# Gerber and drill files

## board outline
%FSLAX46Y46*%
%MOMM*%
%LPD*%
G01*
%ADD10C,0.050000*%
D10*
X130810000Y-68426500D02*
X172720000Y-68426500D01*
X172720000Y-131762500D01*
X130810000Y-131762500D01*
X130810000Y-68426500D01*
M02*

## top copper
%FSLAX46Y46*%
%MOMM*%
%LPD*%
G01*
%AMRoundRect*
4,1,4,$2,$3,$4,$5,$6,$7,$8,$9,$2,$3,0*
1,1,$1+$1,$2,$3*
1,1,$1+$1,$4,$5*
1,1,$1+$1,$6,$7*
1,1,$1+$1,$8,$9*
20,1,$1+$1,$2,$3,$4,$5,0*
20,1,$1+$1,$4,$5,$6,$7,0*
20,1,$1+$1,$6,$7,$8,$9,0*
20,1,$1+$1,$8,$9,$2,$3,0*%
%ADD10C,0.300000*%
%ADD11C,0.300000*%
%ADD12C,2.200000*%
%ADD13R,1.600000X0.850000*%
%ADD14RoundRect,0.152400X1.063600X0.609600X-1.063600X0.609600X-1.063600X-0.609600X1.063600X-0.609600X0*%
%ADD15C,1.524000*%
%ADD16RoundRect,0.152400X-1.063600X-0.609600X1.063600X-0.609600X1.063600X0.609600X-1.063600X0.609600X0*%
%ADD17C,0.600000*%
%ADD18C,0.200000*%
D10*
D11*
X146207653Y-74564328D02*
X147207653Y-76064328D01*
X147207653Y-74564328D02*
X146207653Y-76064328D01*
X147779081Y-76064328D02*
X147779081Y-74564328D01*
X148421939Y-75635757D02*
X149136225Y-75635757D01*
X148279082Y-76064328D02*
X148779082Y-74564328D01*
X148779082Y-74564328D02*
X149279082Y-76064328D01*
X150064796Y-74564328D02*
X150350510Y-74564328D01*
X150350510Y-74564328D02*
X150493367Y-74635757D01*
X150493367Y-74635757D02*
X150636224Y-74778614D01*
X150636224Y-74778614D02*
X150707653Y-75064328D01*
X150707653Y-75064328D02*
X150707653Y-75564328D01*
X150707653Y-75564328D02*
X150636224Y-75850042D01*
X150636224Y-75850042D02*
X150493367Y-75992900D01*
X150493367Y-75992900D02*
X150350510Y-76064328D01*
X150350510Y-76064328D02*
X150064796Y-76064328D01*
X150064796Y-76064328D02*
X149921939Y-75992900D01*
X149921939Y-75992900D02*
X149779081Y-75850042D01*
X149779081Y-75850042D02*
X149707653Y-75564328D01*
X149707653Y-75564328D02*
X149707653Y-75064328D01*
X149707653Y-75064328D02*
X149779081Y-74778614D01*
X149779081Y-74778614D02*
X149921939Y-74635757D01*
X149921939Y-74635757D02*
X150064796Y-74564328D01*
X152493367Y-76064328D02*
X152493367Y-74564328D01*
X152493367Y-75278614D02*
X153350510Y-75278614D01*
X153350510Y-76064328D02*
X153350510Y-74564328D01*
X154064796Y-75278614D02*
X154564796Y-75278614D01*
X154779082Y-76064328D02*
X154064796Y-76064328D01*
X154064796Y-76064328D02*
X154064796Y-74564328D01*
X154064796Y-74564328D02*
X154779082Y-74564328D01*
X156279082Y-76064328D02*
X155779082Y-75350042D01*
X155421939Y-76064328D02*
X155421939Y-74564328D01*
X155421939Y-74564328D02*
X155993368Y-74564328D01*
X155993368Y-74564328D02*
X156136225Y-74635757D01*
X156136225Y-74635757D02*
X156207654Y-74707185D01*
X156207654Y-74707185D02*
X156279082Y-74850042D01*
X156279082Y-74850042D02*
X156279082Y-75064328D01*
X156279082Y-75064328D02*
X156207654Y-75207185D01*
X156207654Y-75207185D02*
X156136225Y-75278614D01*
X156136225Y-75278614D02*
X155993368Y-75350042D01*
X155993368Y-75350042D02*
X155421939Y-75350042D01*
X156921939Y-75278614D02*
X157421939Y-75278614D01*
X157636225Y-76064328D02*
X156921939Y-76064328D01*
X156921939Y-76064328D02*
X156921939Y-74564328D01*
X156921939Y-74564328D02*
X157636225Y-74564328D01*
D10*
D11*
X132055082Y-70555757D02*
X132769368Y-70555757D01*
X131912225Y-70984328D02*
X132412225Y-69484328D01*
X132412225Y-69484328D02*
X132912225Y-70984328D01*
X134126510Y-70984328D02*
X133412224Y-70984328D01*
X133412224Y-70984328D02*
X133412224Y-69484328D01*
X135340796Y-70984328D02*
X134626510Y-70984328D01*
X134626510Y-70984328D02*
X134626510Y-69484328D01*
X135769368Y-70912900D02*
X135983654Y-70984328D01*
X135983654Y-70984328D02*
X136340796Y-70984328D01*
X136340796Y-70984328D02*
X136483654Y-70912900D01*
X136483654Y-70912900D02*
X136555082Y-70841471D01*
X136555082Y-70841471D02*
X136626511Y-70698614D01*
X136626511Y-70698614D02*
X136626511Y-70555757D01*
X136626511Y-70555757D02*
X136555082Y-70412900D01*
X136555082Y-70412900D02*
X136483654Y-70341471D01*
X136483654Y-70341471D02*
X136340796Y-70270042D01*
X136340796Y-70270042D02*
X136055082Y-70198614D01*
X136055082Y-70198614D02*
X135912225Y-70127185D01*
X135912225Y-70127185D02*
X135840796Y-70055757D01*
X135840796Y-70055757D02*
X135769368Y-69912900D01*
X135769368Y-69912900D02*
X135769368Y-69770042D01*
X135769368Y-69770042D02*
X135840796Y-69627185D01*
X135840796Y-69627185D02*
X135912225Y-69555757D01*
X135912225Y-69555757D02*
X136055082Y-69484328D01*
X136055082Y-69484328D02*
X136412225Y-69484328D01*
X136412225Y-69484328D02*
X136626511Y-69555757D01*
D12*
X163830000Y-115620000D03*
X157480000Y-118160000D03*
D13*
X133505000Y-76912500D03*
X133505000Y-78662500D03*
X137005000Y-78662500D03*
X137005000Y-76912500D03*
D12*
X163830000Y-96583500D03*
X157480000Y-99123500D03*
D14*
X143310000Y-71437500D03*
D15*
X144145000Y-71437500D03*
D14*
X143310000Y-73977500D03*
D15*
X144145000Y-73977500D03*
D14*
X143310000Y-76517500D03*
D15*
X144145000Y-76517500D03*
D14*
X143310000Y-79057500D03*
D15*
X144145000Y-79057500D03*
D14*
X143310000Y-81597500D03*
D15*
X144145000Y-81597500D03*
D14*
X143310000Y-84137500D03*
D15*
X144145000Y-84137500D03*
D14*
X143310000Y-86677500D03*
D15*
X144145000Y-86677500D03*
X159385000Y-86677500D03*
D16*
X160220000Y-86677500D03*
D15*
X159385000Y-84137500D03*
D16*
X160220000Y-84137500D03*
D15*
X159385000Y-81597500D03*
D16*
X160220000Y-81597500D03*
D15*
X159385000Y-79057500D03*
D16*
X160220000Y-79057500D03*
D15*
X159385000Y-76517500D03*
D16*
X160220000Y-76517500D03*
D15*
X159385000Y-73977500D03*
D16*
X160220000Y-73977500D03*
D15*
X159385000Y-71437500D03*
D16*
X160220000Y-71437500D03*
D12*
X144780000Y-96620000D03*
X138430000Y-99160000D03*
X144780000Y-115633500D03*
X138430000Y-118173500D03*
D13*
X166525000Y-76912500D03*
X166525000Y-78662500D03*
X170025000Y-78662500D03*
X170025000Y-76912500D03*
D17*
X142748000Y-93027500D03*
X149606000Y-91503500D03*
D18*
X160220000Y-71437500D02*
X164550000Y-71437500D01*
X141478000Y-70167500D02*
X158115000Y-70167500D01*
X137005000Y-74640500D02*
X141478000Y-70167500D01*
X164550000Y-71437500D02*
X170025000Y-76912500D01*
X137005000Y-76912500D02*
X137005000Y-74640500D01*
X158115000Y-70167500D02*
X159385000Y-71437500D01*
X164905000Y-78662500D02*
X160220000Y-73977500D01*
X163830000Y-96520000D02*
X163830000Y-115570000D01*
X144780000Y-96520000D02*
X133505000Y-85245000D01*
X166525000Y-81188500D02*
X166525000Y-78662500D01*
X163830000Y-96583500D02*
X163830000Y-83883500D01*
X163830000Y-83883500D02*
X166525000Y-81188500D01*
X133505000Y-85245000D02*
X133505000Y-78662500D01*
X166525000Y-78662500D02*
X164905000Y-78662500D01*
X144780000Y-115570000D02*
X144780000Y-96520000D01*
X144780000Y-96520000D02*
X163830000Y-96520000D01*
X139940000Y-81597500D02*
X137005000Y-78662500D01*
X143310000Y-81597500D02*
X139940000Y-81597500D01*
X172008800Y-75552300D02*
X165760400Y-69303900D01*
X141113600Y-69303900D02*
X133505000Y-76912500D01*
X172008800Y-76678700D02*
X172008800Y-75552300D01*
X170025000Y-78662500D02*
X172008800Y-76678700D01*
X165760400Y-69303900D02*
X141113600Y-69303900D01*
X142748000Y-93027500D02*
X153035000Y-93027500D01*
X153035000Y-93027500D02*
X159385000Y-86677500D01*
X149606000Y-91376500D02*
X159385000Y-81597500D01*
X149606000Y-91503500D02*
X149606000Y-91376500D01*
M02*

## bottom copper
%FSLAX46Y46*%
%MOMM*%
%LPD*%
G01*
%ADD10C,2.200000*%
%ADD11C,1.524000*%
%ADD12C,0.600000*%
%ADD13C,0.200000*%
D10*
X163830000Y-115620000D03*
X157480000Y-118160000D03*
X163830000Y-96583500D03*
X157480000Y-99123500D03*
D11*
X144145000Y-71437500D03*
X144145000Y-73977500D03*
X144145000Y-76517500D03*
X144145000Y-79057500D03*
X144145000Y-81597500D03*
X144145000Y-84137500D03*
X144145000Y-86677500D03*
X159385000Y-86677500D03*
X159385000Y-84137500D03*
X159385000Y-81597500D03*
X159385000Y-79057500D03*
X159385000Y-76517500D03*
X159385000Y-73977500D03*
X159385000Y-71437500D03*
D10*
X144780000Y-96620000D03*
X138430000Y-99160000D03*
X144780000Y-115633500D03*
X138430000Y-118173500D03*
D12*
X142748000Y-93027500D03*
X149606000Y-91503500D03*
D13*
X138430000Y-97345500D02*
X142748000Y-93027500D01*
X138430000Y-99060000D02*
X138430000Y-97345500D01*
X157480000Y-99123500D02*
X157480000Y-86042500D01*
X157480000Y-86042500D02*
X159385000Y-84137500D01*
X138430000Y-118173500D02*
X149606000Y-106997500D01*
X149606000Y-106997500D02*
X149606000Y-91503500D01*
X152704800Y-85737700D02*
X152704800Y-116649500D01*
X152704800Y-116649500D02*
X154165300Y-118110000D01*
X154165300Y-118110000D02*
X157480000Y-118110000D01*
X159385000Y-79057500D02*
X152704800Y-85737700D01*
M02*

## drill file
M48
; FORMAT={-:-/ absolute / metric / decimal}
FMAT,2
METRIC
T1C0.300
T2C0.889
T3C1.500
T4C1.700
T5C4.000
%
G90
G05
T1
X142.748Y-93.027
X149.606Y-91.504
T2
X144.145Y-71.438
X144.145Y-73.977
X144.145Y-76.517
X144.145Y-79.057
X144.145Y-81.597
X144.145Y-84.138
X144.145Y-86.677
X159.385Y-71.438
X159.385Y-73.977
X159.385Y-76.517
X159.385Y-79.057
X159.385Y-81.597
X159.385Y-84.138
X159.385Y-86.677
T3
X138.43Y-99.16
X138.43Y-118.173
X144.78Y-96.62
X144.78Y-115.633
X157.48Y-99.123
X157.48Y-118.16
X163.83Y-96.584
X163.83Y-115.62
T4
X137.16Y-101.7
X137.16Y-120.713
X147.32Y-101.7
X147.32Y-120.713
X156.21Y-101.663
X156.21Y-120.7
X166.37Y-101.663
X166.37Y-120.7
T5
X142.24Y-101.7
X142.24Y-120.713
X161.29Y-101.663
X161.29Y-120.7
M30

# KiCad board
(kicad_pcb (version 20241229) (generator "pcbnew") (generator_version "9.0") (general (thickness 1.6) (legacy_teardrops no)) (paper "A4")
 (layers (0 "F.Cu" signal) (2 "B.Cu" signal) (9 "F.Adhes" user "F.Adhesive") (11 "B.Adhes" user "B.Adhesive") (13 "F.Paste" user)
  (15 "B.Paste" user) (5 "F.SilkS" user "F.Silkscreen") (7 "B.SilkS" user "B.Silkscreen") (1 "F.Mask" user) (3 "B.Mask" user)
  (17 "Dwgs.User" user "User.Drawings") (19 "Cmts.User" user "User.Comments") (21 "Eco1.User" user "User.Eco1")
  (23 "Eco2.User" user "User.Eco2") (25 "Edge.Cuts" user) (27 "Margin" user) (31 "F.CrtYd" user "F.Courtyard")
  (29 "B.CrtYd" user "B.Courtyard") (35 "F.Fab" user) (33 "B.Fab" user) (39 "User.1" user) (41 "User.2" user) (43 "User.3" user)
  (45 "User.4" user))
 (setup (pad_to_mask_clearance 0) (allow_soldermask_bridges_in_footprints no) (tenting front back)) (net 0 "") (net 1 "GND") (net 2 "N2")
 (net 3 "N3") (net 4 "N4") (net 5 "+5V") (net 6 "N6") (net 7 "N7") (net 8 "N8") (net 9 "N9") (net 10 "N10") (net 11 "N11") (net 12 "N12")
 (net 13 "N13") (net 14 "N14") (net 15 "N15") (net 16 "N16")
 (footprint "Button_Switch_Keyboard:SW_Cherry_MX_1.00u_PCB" (layer "F.Cu") (at 163.83 115.62)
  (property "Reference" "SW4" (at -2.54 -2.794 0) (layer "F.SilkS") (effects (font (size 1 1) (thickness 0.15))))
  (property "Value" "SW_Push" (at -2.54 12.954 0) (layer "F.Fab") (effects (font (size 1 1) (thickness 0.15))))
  (pad "" np_thru_hole circle (at -7.62 5.08) (size 1.7 1.7) (drill 1.7) (layers "*.Cu" "*.Mask"))
  (pad "" np_thru_hole circle (at -2.54 5.08) (size 4 4) (drill 4) (layers "*.Cu" "*.Mask"))
  (pad "" np_thru_hole circle (at 2.54 5.08) (size 1.7 1.7) (drill 1.7) (layers "*.Cu" "*.Mask"))
  (pad "1" thru_hole circle (at 0 0) (size 2.2 2.2) (drill 1.5) (layers "*.Cu" "*.Mask") (remove_unused_layers no) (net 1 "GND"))
  (pad "2" thru_hole circle (at -6.35 2.54) (size 2.2 2.2) (drill 1.5) (layers "*.Cu" "*.Mask") (remove_unused_layers no) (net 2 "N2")))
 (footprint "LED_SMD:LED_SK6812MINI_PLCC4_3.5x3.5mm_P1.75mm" (layer "F.Cu") (at 135.255 77.7875)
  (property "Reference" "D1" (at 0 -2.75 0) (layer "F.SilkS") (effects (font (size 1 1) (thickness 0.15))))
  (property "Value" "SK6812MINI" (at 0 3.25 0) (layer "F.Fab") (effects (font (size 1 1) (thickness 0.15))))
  (pad "1" smd rect (at -1.75 -0.875) (size 1.6 0.85) (layers "F.Cu" "F.Mask" "F.Paste") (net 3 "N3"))
  (pad "2" smd rect (at -1.75 0.875) (size 1.6 0.85) (layers "F.Cu" "F.Mask" "F.Paste") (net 1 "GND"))
  (pad "3" smd rect (at 1.75 0.875) (size 1.6 0.85) (layers "F.Cu" "F.Mask" "F.Paste") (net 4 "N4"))
  (pad "4" smd rect (at 1.75 -0.875) (size 1.6 0.85) (layers "F.Cu" "F.Mask" "F.Paste") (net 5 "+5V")))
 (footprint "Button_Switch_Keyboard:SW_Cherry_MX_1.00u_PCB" (layer "F.Cu") (at 163.83 96.5835)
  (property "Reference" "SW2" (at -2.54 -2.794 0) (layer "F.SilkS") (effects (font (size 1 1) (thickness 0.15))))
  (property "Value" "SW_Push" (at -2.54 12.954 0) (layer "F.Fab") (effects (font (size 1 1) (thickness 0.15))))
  (pad "" np_thru_hole circle (at -7.62 5.08) (size 1.7 1.7) (drill 1.7) (layers "*.Cu" "*.Mask"))
  (pad "" np_thru_hole circle (at -2.54 5.08) (size 4 4) (drill 4) (layers "*.Cu" "*.Mask"))
  (pad "" np_thru_hole circle (at 2.54 5.08) (size 1.7 1.7) (drill 1.7) (layers "*.Cu" "*.Mask"))
  (pad "1" thru_hole circle (at 0 0) (size 2.2 2.2) (drill 1.5) (layers "*.Cu" "*.Mask") (remove_unused_layers no) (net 1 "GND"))
  (pad "2" thru_hole circle (at -6.35 2.54) (size 2.2 2.2) (drill 1.5) (layers "*.Cu" "*.Mask") (remove_unused_layers no) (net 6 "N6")))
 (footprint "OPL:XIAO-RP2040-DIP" (layer "F.Cu") (at 151.765 79.0575)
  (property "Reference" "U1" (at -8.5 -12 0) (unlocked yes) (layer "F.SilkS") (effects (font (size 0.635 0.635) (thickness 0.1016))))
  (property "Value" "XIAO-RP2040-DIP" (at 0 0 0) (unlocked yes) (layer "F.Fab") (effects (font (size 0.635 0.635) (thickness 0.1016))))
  (pad "1" smd roundrect (at -8.455 -7.62 180) (size 2.432 1.524) (layers "F.Cu" "F.Mask") (roundrect_rratio 0.1) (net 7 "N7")
   (thermal_bridge_angle 45))
  (pad "1" thru_hole circle (at -7.62 -7.62 180) (size 1.524 1.524) (drill 0.889) (layers "*.Cu" "*.Mask") (remove_unused_layers no)
   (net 7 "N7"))
  (pad "2" smd roundrect (at -8.455 -5.08 180) (size 2.432 1.524) (layers "F.Cu" "F.Mask") (roundrect_rratio 0.1) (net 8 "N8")
   (thermal_bridge_angle 45))
  (pad "2" thru_hole circle (at -7.62 -5.08 180) (size 1.524 1.524) (drill 0.889) (layers "*.Cu" "*.Mask") (remove_unused_layers no)
   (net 8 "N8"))
  (pad "3" smd roundrect (at -8.455 -2.54 180) (size 2.432 1.524) (layers "F.Cu" "F.Mask") (roundrect_rratio 0.1) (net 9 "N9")
   (thermal_bridge_angle 45))
  (pad "3" thru_hole circle (at -7.62 -2.54 180) (size 1.524 1.524) (drill 0.889) (layers "*.Cu" "*.Mask") (remove_unused_layers no)
   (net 9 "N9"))
  (pad "4" smd roundrect (at -8.455 0 180) (size 2.432 1.524) (layers "F.Cu" "F.Mask") (roundrect_rratio 0.1) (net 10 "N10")
   (thermal_bridge_angle 45))
  (pad "4" thru_hole circle (at -7.62 0 180) (size 1.524 1.524) (drill 0.889) (layers "*.Cu" "*.Mask") (remove_unused_layers no)
   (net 10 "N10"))
  (pad "5" smd roundrect (at -8.455 2.54 180) (size 2.432 1.524) (layers "F.Cu" "F.Mask") (roundrect_rratio 0.1) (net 4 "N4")
   (thermal_bridge_angle 45))
  (pad "5" thru_hole circle (at -7.62 2.54 180) (size 1.524 1.524) (drill 0.889) (layers "*.Cu" "*.Mask") (remove_unused_layers no)
   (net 4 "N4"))
  (pad "6" smd roundrect (at -8.455 5.08 180) (size 2.432 1.524) (layers "F.Cu" "F.Mask") (roundrect_rratio 0.1) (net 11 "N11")
   (thermal_bridge_angle 45))
  (pad "6" thru_hole circle (at -7.62 5.08 180) (size 1.524 1.524) (drill 0.889) (layers "*.Cu" "*.Mask") (remove_unused_layers no)
   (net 11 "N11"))
  (pad "7" smd roundrect (at -8.455 7.62 180) (size 2.432 1.524) (layers "F.Cu" "F.Mask") (roundrect_rratio 0.1) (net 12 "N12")
   (thermal_bridge_angle 45))
  (pad "7" thru_hole circle (at -7.62 7.62 180) (size 1.524 1.524) (drill 0.889) (layers "*.Cu" "*.Mask") (remove_unused_layers no)
   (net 12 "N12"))
  (pad "8" thru_hole circle (at 7.62 7.62) (size 1.524 1.524) (drill 0.889) (layers "*.Cu" "*.Mask") (remove_unused_layers no)
   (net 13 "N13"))
  (pad "8" smd roundrect (at 8.455 7.62) (size 2.432 1.524) (layers "F.Cu" "F.Mask") (roundrect_rratio 0.1) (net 13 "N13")
   (thermal_bridge_angle 45))
  (pad "9" thru_hole circle (at 7.62 5.08) (size 1.524 1.524) (drill 0.889) (layers "*.Cu" "*.Mask") (remove_unused_layers no) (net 6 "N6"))
  (pad "9" smd roundrect (at 8.455 5.08) (size 2.432 1.524) (layers "F.Cu" "F.Mask") (roundrect_rratio 0.1) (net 6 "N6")
   (thermal_bridge_angle 45))
  (pad "10" thru_hole circle (at 7.62 2.54) (size 1.524 1.524) (drill 0.889) (layers "*.Cu" "*.Mask") (remove_unused_layers no)
   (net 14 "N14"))
  (pad "10" smd roundrect (at 8.455 2.54) (size 2.432 1.524) (layers "F.Cu" "F.Mask") (roundrect_rratio 0.1) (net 14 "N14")
   (thermal_bridge_angle 45))
  (pad "11" thru_hole circle (at 7.62 0) (size 1.524 1.524) (drill 0.889) (layers "*.Cu" "*.Mask") (remove_unused_layers no) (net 2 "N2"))
  (pad "11" smd roundrect (at 8.455 0) (size 2.432 1.524) (layers "F.Cu" "F.Mask") (roundrect_rratio 0.1) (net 2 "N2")
   (thermal_bridge_angle 45))
  (pad "12" thru_hole circle (at 7.62 -2.54) (size 1.524 1.524) (drill 0.889) (layers "*.Cu" "*.Mask") (remove_unused_layers no)
   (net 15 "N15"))
  (pad "12" smd roundrect (at 8.455 -2.54) (size 2.432 1.524) (layers "F.Cu" "F.Mask") (roundrect_rratio 0.1) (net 15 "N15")
   (thermal_bridge_angle 45))
  (pad "13" thru_hole circle (at 7.62 -5.08) (size 1.524 1.524) (drill 0.889) (layers "*.Cu" "*.Mask") (remove_unused_layers no)
   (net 1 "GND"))
  (pad "13" smd roundrect (at 8.455 -5.08) (size 2.432 1.524) (layers "F.Cu" "F.Mask") (roundrect_rratio 0.1) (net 1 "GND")
   (thermal_bridge_angle 45))
  (pad "14" thru_hole circle (at 7.62 -7.62) (size 1.524 1.524) (drill 0.889) (layers "*.Cu" "*.Mask") (remove_unused_layers no)
   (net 5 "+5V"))
  (pad "14" smd roundrect (at 8.455 -7.62) (size 2.432 1.524) (layers "F.Cu" "F.Mask") (roundrect_rratio 0.1) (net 5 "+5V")
   (thermal_bridge_angle 45)))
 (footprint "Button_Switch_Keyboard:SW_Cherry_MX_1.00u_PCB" (layer "F.Cu") (at 144.78 96.62)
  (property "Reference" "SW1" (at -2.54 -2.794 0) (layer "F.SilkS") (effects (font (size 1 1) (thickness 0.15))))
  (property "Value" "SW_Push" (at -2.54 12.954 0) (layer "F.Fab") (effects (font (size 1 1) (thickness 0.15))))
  (pad "" np_thru_hole circle (at -7.62 5.08) (size 1.7 1.7) (drill 1.7) (layers "*.Cu" "*.Mask"))
  (pad "" np_thru_hole circle (at -2.54 5.08) (size 4 4) (drill 4) (layers "*.Cu" "*.Mask"))
  (pad "" np_thru_hole circle (at 2.54 5.08) (size 1.7 1.7) (drill 1.7) (layers "*.Cu" "*.Mask"))
  (pad "1" thru_hole circle (at 0 0) (size 2.2 2.2) (drill 1.5) (layers "*.Cu" "*.Mask") (remove_unused_layers no) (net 1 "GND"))
  (pad "2" thru_hole circle (at -6.35 2.54) (size 2.2 2.2) (drill 1.5) (layers "*.Cu" "*.Mask") (remove_unused_layers no) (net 13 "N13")))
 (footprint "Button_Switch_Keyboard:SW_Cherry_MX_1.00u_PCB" (layer "F.Cu") (at 144.78 115.6335)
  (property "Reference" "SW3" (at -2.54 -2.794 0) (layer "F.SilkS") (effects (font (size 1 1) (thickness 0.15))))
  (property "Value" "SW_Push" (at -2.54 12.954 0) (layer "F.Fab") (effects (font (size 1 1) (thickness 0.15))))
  (pad "" np_thru_hole circle (at -7.62 5.08) (size 1.7 1.7) (drill 1.7) (layers "*.Cu" "*.Mask"))
  (pad "" np_thru_hole circle (at -2.54 5.08) (size 4 4) (drill 4) (layers "*.Cu" "*.Mask"))
  (pad "" np_thru_hole circle (at 2.54 5.08) (size 1.7 1.7) (drill 1.7) (layers "*.Cu" "*.Mask"))
  (pad "1" thru_hole circle (at 0 0) (size 2.2 2.2) (drill 1.5) (layers "*.Cu" "*.Mask") (remove_unused_layers no) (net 1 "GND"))
  (pad "2" thru_hole circle (at -6.35 2.54) (size 2.2 2.2) (drill 1.5) (layers "*.Cu" "*.Mask") (remove_unused_layers no) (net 14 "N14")))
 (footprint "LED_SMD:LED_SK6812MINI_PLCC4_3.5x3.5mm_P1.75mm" (layer "F.Cu") (at 168.275 77.7875)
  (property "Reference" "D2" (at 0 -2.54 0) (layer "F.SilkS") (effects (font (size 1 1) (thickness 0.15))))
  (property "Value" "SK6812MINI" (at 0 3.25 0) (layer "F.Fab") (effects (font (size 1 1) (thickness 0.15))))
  (pad "1" smd rect (at -1.75 -0.875) (size 1.6 0.85) (layers "F.Cu" "F.Mask" "F.Paste") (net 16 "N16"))
  (pad "2" smd rect (at -1.75 0.875) (size 1.6 0.85) (layers "F.Cu" "F.Mask" "F.Paste") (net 1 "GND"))
  (pad "3" smd rect (at 1.75 0.875) (size 1.6 0.85) (layers "F.Cu" "F.Mask" "F.Paste") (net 3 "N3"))
  (pad "4" smd rect (at 1.75 -0.875) (size 1.6 0.85) (layers "F.Cu" "F.Mask" "F.Paste") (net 5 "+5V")))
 (gr_rect (start 130.81 68.4265) (end 172.72 131.7625) (stroke (width 0.05) (type default)) (fill no) (layer "Edge.Cuts"))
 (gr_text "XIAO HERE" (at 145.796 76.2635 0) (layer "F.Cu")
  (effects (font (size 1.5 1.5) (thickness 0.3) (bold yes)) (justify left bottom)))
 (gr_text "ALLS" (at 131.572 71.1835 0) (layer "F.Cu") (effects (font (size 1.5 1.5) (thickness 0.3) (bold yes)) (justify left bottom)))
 (segment (start 160.22 71.4375) (end 164.55 71.4375) (width 0.2) (layer "F.Cu") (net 5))
 (segment (start 141.478 70.1675) (end 158.115 70.1675) (width 0.2) (layer "F.Cu") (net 5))
 (segment (start 137.005 74.6405) (end 141.478 70.1675) (width 0.2) (layer "F.Cu") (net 5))
 (segment (start 164.55 71.4375) (end 170.025 76.9125) (width 0.2) (layer "F.Cu") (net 5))
 (segment (start 137.005 76.9125) (end 137.005 74.6405) (width 0.2) (layer "F.Cu") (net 5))
 (segment (start 158.115 70.1675) (end 159.385 71.4375) (width 0.2) (layer "F.Cu") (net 5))
 (segment (start 164.905 78.6625) (end 160.22 73.9775) (width 0.2) (layer "F.Cu") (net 1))
 (segment (start 163.83 96.52) (end 163.83 115.57) (width 0.2) (layer "F.Cu") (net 1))
 (segment (start 144.78 96.52) (end 133.505 85.245) (width 0.2) (layer "F.Cu") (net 1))
 (segment (start 166.525 81.1885) (end 166.525 78.6625) (width 0.2) (layer "F.Cu") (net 1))
 (segment (start 163.83 96.5835) (end 163.83 83.8835) (width 0.2) (layer "F.Cu") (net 1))
 (segment (start 163.83 83.8835) (end 166.525 81.1885) (width 0.2) (layer "F.Cu") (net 1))
 (segment (start 133.505 85.245) (end 133.505 78.6625) (width 0.2) (layer "F.Cu") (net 1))
 (segment (start 166.525 78.6625) (end 164.905 78.6625) (width 0.2) (layer "F.Cu") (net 1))
 (segment (start 144.78 115.57) (end 144.78 96.52) (width 0.2) (layer "F.Cu") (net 1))
 (segment (start 144.78 96.52) (end 163.83 96.52) (width 0.2) (layer "F.Cu") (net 1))
 (segment (start 139.94 81.5975) (end 137.005 78.6625) (width 0.2) (layer "F.Cu") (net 4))
 (segment (start 143.31 81.5975) (end 139.94 81.5975) (width 0.2) (layer "F.Cu") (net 4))
 (segment (start 172.0088 75.5523) (end 165.7604 69.3039) (width 0.2) (layer "F.Cu") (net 3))
 (segment (start 141.1136 69.3039) (end 133.505 76.9125) (width 0.2) (layer "F.Cu") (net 3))
 (segment (start 172.0088 76.6787) (end 172.0088 75.5523) (width 0.2) (layer "F.Cu") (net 3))
 (segment (start 170.025 78.6625) (end 172.0088 76.6787) (width 0.2) (layer "F.Cu") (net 3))
 (segment (start 165.7604 69.3039) (end 141.1136 69.3039) (width 0.2) (layer "F.Cu") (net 3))
 (segment (start 142.748 93.0275) (end 153.035 93.0275) (width 0.2) (layer "F.Cu") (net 13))
 (segment (start 153.035 93.0275) (end 159.385 86.6775) (width 0.2) (layer "F.Cu") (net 13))
 (via (at 142.748 93.0275) (size 0.6) (drill 0.3) (layers "F.Cu" "B.Cu") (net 13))
 (segment (start 138.43 97.3455) (end 142.748 93.0275) (width 0.2) (layer "B.Cu") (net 13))
 (segment (start 138.43 99.06) (end 138.43 97.3455) (width 0.2) (layer "B.Cu") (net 13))
 (segment (start 157.48 99.1235) (end 157.48 86.0425) (width 0.2) (layer "B.Cu") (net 6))
 (segment (start 157.48 86.0425) (end 159.385 84.1375) (width 0.2) (layer "B.Cu") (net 6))
 (segment (start 149.606 91.3765) (end 159.385 81.5975) (width 0.2) (layer "F.Cu") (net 14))
 (segment (start 149.606 91.5035) (end 149.606 91.3765) (width 0.2) (layer "F.Cu") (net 14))
 (via (at 149.606 91.5035) (size 0.6) (drill 0.3) (layers "F.Cu" "B.Cu") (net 14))
 (segment (start 138.43 118.1735) (end 149.606 106.9975) (width 0.2) (layer "B.Cu") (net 14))
 (segment (start 149.606 106.9975) (end 149.606 91.5035) (width 0.2) (layer "B.Cu") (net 14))
 (segment (start 152.7048 85.7377) (end 152.7048 116.6495) (width 0.2) (layer "B.Cu") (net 2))
 (segment (start 152.7048 116.6495) (end 154.1653 118.11) (width 0.2) (layer "B.Cu") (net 2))
 (segment (start 154.1653 118.11) (end 157.48 118.11) (width 0.2) (layer "B.Cu") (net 2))
 (segment (start 159.385 79.0575) (end 152.7048 85.7377) (width 0.2) (layer "B.Cu") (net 2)))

